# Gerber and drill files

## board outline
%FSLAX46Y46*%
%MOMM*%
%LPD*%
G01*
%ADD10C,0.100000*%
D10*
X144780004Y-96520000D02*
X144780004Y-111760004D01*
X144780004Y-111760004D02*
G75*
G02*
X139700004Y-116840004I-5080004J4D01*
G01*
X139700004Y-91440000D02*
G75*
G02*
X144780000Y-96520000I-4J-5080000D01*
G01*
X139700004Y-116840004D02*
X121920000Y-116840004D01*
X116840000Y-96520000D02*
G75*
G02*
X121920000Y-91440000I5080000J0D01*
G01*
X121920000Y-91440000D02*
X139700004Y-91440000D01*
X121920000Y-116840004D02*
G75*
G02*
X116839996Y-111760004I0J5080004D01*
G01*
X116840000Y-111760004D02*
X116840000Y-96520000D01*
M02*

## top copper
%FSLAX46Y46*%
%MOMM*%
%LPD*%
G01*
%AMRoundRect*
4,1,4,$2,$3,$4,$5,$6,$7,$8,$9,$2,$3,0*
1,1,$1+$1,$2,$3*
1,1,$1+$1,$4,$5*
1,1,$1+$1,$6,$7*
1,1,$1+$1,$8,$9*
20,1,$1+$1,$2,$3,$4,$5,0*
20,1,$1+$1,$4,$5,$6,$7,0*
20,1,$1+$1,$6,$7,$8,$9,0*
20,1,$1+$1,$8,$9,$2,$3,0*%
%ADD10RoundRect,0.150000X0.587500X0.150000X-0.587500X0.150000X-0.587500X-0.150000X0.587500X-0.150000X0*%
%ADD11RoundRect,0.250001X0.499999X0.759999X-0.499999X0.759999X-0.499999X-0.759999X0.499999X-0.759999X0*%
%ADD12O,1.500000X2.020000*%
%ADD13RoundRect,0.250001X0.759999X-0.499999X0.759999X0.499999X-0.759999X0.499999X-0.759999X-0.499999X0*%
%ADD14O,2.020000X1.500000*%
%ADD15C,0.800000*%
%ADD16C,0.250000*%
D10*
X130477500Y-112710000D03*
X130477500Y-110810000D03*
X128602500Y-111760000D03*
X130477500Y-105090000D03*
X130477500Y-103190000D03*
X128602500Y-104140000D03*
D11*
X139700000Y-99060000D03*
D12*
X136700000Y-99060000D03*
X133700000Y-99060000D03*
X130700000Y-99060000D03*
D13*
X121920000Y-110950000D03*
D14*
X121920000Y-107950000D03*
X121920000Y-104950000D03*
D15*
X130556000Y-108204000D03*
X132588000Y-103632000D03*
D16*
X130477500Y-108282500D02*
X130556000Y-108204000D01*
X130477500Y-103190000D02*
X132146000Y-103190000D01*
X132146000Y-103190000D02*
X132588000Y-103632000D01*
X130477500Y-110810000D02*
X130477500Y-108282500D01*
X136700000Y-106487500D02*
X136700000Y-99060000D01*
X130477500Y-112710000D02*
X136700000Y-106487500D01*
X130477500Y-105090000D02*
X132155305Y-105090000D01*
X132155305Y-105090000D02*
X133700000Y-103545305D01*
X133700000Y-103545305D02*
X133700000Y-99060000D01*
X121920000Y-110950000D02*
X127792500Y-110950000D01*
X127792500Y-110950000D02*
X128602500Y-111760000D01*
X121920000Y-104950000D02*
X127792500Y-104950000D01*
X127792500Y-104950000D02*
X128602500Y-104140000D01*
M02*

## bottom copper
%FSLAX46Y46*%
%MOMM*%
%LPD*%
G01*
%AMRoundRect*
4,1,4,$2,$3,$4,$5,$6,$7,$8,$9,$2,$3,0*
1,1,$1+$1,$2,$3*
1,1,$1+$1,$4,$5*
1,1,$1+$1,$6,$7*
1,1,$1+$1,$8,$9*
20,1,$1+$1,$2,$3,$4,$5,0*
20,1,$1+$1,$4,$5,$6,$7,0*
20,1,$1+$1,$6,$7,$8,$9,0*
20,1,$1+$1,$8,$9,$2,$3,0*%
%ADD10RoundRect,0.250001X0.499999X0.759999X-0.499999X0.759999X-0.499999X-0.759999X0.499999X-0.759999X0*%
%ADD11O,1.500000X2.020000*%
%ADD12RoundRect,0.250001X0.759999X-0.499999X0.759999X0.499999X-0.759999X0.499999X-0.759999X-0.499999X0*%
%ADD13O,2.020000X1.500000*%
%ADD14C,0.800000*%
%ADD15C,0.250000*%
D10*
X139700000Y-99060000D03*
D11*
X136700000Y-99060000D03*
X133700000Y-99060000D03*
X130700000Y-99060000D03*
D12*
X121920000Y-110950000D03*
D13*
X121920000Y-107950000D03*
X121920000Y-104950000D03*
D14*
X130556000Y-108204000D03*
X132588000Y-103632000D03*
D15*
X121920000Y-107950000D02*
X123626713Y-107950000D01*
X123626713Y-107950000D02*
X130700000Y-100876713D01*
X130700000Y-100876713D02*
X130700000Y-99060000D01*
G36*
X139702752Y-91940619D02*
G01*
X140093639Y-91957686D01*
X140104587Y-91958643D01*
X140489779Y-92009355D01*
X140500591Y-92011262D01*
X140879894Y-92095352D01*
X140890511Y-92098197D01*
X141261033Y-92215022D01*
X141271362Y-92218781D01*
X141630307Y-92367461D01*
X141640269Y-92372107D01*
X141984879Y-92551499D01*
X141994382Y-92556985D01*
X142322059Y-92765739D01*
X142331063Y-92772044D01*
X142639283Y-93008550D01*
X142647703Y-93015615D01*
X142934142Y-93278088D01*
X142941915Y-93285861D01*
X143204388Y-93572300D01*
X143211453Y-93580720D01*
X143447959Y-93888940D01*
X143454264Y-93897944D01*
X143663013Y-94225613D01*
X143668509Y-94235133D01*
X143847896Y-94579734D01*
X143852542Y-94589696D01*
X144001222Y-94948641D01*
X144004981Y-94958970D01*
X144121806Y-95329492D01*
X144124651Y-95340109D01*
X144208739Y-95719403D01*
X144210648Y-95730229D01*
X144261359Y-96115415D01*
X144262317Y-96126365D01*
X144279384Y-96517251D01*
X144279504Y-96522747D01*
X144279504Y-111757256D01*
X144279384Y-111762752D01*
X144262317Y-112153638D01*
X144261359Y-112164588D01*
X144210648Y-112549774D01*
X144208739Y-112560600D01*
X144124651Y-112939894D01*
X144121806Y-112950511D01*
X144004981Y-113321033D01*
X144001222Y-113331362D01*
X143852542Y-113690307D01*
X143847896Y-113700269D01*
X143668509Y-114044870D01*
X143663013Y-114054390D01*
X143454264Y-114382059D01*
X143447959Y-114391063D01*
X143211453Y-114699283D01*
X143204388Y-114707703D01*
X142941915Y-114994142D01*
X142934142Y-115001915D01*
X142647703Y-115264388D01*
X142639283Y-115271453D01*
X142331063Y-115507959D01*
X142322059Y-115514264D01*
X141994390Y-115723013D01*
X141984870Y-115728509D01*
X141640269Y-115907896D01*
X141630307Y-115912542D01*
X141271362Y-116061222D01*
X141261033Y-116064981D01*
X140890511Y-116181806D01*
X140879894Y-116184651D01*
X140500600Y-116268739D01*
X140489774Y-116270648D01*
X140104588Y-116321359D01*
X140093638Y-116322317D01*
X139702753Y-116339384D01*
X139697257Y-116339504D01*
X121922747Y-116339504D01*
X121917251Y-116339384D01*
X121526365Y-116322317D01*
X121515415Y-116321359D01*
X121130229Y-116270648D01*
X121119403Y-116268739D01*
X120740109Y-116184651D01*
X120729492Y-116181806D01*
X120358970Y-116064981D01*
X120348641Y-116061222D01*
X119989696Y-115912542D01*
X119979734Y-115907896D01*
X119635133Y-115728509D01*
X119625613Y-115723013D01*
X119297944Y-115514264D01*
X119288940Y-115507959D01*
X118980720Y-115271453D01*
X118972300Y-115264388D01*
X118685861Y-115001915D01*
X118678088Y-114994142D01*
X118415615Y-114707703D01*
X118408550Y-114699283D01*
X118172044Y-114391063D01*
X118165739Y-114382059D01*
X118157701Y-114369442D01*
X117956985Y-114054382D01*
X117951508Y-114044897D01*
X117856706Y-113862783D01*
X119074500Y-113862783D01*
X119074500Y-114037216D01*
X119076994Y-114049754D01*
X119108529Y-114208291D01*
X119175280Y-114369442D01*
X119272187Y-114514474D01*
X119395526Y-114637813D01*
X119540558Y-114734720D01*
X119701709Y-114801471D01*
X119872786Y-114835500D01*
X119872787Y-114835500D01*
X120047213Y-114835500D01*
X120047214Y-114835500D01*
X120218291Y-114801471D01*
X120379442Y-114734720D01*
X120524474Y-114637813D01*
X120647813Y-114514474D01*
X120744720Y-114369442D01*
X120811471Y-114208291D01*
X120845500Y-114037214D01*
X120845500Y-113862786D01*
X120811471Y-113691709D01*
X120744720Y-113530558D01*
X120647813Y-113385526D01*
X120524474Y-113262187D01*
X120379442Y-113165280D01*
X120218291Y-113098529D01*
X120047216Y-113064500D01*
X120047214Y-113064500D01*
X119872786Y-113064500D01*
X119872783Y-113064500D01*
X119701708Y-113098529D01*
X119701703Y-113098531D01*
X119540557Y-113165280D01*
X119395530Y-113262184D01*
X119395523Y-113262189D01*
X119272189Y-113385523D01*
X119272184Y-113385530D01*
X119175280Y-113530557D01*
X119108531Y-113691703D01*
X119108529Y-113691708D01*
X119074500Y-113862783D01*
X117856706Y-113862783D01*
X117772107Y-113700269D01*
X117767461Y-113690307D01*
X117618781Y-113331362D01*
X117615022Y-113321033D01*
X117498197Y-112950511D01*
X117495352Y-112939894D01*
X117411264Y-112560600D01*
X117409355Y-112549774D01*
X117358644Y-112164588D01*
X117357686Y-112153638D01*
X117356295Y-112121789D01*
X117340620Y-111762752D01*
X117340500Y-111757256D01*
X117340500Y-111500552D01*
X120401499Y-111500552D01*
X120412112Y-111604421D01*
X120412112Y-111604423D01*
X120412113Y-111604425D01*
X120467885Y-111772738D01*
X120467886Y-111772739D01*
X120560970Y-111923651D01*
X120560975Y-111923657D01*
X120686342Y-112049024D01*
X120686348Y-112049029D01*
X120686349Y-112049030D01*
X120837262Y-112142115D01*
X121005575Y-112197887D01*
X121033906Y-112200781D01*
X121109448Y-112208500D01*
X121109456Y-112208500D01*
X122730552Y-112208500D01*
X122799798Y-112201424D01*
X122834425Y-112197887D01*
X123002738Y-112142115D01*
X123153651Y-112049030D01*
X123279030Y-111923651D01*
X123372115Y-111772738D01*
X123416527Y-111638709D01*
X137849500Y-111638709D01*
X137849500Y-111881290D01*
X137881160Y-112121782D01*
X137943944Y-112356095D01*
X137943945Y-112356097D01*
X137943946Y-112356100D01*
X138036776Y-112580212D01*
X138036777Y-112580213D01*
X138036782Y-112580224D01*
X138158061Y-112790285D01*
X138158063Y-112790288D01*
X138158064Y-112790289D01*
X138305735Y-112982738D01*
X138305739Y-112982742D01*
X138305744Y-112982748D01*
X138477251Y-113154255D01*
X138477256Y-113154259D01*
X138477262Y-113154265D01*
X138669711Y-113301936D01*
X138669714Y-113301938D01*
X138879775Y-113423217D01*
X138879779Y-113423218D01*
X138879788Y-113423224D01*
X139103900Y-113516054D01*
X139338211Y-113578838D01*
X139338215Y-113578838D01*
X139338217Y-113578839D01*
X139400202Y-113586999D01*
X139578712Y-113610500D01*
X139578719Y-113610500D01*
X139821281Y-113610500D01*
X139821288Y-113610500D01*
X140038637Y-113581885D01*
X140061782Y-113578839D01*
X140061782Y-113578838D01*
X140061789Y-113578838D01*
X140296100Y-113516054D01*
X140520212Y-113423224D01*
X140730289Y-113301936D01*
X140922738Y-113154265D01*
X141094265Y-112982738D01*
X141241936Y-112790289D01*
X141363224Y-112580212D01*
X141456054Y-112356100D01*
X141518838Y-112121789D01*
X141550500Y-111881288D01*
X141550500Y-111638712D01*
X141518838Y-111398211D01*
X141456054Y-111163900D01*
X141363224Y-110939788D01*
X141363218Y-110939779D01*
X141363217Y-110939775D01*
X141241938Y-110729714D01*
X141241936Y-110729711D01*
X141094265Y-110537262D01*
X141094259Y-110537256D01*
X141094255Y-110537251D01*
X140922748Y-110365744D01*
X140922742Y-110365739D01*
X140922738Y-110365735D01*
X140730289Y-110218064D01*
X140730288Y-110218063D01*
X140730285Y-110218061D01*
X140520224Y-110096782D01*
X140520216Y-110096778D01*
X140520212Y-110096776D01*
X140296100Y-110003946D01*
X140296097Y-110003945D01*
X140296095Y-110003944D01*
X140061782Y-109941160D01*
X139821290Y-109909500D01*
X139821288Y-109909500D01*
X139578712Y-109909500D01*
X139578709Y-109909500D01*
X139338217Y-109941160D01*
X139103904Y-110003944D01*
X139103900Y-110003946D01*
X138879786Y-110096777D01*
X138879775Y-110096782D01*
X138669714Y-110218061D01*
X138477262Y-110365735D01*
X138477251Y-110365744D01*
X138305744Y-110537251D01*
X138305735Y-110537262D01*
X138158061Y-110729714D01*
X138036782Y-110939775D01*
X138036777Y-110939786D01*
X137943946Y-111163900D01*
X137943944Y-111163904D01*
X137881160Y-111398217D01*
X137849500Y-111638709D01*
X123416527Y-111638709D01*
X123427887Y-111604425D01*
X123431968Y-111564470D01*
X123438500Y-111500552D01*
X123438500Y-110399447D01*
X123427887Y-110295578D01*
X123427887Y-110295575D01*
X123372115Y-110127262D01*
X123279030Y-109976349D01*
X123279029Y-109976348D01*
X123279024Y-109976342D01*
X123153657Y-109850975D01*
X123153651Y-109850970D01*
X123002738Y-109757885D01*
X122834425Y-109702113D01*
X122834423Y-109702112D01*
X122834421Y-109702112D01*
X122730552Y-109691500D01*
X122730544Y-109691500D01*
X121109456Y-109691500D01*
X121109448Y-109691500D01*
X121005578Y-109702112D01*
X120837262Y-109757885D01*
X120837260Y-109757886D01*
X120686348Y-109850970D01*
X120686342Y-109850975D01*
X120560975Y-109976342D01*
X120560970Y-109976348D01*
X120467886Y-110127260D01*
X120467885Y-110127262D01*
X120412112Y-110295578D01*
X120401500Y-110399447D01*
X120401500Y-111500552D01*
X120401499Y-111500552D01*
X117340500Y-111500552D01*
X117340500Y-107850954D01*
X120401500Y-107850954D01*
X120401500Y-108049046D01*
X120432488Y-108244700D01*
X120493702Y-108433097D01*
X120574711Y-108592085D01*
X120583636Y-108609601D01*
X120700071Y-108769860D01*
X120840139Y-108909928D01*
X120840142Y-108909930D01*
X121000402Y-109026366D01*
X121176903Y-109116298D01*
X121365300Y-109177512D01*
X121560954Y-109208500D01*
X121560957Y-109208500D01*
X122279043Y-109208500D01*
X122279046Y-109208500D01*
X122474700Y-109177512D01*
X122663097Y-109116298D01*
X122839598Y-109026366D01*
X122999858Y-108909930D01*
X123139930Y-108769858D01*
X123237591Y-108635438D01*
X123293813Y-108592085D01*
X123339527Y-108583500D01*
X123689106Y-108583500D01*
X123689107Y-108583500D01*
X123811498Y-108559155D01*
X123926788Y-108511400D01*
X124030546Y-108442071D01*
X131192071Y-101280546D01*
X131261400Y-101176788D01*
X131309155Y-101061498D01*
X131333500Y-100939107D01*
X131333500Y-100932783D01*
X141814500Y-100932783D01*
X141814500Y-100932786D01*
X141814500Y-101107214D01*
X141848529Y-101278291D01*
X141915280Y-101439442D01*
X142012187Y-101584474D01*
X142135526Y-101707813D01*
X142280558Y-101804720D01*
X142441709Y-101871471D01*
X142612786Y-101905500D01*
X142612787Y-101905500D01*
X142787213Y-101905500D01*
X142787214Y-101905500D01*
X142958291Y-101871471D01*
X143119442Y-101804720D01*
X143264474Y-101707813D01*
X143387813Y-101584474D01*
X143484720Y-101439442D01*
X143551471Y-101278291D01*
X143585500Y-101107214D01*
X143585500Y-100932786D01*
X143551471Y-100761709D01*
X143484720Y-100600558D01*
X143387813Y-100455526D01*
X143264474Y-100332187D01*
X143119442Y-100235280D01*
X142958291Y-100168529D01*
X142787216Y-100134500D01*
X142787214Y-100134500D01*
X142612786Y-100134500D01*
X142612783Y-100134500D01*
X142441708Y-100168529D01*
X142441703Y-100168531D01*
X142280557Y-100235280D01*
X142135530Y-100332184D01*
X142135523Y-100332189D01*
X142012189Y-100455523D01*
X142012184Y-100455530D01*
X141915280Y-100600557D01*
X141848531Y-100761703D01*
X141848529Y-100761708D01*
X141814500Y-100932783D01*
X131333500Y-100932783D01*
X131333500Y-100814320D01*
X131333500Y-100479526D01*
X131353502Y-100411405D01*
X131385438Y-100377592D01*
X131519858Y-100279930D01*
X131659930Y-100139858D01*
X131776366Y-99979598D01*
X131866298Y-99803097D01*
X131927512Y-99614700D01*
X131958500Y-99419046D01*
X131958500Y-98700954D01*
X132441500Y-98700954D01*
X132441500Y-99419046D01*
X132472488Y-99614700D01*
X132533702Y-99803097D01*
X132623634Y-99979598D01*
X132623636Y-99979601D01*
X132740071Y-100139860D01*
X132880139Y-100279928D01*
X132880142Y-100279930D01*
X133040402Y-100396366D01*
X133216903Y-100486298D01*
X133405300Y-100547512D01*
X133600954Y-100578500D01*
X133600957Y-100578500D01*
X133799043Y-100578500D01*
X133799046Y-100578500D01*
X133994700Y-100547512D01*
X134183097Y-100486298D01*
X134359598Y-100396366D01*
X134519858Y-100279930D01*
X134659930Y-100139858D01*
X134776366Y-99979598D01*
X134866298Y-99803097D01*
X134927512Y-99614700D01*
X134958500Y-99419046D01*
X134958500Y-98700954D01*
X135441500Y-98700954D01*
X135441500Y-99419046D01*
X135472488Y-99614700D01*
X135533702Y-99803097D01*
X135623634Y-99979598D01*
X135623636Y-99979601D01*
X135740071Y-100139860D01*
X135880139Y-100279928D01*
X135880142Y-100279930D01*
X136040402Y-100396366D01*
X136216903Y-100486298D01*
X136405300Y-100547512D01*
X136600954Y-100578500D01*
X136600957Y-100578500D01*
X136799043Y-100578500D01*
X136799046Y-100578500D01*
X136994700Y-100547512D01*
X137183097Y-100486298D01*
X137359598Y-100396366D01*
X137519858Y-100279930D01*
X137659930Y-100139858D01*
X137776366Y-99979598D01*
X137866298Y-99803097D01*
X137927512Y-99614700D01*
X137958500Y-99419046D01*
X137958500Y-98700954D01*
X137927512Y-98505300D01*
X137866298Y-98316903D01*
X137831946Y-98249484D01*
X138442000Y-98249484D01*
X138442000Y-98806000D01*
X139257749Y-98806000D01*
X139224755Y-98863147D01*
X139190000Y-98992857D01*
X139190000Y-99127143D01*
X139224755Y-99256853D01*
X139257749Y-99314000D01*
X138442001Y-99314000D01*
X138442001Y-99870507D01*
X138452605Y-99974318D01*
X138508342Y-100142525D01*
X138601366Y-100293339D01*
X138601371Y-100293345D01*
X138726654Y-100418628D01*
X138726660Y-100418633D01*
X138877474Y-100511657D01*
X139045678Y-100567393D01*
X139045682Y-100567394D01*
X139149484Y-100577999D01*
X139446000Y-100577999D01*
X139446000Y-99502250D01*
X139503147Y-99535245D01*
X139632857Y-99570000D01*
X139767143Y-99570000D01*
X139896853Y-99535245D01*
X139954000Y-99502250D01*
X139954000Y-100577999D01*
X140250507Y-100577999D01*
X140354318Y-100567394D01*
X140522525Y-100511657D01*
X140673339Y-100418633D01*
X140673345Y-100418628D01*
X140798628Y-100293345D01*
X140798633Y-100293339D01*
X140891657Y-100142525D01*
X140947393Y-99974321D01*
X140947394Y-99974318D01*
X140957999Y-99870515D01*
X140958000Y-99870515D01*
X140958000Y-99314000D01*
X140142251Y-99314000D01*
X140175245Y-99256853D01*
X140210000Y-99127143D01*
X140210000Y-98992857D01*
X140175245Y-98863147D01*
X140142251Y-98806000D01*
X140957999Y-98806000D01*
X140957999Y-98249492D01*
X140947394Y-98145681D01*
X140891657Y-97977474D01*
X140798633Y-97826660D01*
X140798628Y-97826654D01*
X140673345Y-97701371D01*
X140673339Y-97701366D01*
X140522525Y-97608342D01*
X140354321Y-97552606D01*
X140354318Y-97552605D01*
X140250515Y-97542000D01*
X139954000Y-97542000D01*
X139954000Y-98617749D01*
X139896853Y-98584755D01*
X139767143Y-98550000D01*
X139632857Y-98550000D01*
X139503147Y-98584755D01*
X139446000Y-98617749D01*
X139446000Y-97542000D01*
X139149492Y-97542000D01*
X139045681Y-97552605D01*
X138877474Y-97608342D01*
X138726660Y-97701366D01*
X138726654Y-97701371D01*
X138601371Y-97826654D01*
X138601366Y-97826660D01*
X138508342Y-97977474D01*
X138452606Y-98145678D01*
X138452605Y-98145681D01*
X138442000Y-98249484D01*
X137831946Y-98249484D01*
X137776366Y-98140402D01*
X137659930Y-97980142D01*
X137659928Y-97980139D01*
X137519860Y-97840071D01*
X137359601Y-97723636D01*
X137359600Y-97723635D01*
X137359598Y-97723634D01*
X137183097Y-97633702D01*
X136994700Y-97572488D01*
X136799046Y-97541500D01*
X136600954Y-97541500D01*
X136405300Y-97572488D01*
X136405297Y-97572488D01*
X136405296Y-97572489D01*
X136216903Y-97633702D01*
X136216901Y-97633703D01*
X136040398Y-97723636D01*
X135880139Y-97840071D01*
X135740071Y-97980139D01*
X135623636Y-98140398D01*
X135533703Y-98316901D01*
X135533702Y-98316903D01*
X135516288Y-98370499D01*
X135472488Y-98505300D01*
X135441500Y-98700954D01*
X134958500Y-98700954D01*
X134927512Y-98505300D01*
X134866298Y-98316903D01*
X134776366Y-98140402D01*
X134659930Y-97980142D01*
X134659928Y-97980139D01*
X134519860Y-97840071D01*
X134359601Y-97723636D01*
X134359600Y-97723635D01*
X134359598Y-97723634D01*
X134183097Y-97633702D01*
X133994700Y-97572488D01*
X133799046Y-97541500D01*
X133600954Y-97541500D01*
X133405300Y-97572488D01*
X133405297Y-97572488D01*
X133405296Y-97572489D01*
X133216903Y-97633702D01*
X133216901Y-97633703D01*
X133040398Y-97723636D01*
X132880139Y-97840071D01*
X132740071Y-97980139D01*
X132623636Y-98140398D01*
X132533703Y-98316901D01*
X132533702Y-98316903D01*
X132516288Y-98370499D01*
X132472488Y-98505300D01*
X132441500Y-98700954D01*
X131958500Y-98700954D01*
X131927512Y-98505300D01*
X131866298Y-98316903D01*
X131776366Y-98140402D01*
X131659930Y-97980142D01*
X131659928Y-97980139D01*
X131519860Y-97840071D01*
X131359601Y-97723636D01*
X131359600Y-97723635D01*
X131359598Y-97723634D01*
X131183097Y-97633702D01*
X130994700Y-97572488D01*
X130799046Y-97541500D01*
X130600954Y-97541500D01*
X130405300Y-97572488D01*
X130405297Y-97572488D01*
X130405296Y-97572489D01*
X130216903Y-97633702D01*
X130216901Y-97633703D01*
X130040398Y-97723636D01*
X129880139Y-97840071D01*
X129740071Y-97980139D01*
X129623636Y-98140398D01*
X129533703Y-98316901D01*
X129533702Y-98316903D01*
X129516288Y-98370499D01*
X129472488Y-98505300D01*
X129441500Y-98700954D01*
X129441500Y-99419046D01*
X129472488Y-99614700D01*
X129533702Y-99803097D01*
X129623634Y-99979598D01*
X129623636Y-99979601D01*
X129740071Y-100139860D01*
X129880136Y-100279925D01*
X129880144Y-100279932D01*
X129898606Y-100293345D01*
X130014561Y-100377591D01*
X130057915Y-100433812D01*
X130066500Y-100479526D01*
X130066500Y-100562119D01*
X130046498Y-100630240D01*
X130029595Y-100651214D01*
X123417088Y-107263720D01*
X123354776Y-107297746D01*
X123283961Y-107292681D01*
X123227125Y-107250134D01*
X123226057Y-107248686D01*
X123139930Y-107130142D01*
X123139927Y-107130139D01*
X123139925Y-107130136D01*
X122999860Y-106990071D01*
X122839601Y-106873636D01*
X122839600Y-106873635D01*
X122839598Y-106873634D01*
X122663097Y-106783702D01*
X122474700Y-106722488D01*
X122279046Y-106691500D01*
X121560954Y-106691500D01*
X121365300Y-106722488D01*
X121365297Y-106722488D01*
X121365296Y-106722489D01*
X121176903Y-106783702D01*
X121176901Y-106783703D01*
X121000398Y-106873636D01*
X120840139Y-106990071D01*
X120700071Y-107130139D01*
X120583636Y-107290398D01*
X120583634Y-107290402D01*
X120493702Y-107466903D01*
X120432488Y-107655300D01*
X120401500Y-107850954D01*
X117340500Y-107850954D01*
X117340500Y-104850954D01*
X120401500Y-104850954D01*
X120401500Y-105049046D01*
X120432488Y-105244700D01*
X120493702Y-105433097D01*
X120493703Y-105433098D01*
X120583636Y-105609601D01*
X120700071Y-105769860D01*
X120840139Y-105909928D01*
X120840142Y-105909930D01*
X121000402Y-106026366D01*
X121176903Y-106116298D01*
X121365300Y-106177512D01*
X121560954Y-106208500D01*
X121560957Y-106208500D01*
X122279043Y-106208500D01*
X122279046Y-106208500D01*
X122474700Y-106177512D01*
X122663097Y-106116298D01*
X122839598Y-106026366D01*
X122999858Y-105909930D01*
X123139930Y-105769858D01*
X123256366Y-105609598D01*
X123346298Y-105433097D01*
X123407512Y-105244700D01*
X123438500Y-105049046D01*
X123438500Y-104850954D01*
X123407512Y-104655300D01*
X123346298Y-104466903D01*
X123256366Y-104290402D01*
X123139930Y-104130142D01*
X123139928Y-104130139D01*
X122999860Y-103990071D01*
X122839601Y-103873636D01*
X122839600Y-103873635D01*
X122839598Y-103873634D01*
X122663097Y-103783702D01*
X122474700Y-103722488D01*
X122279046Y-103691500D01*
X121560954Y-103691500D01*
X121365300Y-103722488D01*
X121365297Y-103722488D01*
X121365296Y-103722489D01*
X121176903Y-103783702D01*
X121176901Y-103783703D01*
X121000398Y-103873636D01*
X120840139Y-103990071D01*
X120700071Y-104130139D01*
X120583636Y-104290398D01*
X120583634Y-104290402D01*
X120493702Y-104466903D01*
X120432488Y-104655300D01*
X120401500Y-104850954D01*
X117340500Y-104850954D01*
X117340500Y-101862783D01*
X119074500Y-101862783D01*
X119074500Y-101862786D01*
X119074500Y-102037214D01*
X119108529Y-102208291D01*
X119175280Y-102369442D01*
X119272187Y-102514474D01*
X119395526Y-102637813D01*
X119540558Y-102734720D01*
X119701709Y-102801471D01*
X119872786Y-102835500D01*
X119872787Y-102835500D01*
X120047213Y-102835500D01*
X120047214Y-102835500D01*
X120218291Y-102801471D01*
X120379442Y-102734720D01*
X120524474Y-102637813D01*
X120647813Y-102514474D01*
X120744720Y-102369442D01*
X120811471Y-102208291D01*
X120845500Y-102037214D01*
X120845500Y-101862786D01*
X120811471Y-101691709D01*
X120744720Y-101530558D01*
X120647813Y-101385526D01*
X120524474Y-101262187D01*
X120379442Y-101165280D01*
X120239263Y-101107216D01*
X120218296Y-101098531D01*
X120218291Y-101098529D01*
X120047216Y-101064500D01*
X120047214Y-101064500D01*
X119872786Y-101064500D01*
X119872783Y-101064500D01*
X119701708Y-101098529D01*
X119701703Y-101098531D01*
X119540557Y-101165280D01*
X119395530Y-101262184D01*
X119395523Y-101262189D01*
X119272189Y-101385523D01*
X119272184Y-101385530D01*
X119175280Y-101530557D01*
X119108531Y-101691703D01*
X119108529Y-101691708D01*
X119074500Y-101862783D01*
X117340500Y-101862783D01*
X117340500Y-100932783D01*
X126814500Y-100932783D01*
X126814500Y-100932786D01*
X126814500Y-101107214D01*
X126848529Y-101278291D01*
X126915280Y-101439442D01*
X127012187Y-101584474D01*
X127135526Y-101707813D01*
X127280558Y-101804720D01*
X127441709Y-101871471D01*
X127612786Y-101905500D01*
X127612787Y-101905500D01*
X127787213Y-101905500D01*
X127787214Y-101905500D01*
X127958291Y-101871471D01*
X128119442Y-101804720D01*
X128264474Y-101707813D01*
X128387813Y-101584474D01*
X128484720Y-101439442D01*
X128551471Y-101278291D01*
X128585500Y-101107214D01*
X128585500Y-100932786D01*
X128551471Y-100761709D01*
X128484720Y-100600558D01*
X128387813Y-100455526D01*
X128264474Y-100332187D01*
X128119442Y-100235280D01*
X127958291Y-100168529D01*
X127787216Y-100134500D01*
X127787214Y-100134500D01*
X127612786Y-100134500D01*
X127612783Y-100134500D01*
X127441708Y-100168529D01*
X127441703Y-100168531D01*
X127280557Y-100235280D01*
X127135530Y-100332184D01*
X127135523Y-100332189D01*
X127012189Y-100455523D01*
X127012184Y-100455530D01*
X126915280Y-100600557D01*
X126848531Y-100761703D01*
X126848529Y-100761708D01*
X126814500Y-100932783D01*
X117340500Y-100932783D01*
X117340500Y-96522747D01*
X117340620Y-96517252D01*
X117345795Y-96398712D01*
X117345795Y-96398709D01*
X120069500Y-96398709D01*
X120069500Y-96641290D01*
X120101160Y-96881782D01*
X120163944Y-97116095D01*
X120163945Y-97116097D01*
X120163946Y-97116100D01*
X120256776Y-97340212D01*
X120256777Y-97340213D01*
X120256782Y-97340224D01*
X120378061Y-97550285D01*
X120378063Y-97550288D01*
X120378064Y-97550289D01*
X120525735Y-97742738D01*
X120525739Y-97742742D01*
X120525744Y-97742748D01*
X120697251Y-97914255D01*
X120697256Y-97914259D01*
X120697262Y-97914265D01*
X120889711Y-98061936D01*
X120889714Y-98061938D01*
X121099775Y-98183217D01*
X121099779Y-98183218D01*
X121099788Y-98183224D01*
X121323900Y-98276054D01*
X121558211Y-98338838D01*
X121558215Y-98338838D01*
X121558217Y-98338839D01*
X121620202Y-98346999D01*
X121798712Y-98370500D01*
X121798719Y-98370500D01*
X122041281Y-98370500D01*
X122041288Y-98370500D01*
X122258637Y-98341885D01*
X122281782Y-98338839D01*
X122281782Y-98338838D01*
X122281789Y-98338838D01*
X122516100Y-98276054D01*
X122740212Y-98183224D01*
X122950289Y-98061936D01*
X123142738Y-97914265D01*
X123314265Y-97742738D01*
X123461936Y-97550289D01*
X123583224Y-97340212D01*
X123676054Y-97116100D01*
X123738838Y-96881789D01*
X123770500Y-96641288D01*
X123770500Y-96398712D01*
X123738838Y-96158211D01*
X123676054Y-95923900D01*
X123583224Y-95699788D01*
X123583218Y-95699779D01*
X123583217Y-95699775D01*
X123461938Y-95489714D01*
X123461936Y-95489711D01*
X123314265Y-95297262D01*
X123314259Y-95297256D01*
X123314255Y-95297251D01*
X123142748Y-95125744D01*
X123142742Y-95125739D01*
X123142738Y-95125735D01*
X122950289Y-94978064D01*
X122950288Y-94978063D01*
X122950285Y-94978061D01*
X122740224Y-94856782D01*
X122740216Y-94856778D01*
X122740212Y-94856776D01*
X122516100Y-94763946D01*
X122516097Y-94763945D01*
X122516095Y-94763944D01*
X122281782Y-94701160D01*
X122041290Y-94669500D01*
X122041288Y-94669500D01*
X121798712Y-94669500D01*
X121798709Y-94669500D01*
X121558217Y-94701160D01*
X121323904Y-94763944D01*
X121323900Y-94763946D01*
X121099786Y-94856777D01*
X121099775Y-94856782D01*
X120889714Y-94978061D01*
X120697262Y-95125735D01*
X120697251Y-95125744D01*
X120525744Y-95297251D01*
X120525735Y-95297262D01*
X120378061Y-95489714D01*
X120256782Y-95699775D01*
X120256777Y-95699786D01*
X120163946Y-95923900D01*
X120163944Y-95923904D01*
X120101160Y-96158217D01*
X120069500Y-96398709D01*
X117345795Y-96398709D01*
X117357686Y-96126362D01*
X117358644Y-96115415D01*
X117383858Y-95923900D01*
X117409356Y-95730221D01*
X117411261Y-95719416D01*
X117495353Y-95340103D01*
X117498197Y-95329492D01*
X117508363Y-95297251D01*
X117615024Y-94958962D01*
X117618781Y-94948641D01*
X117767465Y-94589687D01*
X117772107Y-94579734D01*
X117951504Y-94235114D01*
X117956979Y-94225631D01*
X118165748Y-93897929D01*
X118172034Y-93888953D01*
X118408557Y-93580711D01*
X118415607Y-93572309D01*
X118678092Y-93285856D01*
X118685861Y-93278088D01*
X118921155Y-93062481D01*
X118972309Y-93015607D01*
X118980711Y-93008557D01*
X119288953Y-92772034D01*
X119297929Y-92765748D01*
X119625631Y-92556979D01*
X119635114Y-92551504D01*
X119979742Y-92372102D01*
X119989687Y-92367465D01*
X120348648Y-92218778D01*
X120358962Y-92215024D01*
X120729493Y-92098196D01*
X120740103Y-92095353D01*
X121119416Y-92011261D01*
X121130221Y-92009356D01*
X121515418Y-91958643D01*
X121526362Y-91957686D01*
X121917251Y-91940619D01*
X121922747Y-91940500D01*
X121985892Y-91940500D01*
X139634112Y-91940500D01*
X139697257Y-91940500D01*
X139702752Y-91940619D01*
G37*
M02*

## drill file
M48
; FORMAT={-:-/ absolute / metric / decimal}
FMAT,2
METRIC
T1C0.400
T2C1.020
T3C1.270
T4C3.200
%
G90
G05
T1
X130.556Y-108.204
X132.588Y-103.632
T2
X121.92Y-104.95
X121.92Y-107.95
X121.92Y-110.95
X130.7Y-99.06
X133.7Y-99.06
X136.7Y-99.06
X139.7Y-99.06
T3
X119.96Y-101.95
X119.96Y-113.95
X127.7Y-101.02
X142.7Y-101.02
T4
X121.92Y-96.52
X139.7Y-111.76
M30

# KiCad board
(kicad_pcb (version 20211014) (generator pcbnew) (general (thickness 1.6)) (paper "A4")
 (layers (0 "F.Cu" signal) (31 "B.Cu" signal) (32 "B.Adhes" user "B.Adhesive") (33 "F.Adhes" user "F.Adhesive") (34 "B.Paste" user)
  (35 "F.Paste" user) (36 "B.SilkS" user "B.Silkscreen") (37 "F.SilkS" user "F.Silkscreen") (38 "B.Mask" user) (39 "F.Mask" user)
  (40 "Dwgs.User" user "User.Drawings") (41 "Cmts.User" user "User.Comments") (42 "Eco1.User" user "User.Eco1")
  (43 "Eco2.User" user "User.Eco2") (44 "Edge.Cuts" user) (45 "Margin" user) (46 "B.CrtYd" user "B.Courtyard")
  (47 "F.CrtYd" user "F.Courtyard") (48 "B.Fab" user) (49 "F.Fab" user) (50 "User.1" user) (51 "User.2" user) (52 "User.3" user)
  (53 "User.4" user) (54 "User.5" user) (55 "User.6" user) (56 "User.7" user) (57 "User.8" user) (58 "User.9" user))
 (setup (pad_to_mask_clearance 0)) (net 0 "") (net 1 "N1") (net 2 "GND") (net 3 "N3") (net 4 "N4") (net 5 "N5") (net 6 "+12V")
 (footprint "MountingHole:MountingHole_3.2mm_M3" (layer "F.Cu") (at 139.7 111.76)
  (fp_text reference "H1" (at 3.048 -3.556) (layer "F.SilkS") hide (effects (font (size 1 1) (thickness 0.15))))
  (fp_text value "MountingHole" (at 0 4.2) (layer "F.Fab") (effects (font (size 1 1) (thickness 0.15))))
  (pad "" np_thru_hole circle (at 0 0) (size 3.2 3.2) (drill 3.2) (layers *.Cu *.Mask)))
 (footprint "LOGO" (layer "F.Cu") (at 139.3698 105.0036)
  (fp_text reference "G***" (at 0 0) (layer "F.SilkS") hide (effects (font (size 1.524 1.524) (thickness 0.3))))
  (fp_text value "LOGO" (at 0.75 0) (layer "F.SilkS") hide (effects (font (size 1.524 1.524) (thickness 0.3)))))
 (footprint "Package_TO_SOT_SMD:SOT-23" (layer "F.Cu") (at 129.54 111.76 180)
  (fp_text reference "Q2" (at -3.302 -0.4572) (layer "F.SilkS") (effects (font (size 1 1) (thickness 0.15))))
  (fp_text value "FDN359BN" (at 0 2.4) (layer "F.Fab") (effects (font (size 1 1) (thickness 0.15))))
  (pad "1" smd roundrect (at -0.9375 -0.95 180) (size 1.475 0.6) (layers "F.Cu" "F.Paste" "F.Mask") (roundrect_rratio 0.25) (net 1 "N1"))
  (pad "2" smd roundrect (at -0.9375 0.95 180) (size 1.475 0.6) (layers "F.Cu" "F.Paste" "F.Mask") (roundrect_rratio 0.25) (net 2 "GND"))
  (pad "3" smd roundrect (at 0.9375 0 180) (size 1.475 0.6) (layers "F.Cu" "F.Paste" "F.Mask") (roundrect_rratio 0.25) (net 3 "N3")))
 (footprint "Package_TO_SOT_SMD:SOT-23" (layer "F.Cu") (at 129.54 104.14 180)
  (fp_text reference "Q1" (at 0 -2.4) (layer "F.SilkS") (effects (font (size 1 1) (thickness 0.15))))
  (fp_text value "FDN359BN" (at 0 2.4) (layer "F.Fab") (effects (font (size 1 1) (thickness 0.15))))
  (pad "1" smd roundrect (at -0.9375 -0.95 180) (size 1.475 0.6) (layers "F.Cu" "F.Paste" "F.Mask") (roundrect_rratio 0.25) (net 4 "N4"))
  (pad "2" smd roundrect (at -0.9375 0.95 180) (size 1.475 0.6) (layers "F.Cu" "F.Paste" "F.Mask") (roundrect_rratio 0.25) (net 2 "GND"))
  (pad "3" smd roundrect (at 0.9375 0 180) (size 1.475 0.6) (layers "F.Cu" "F.Paste" "F.Mask") (roundrect_rratio 0.25) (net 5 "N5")))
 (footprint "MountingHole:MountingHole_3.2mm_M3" (layer "F.Cu") (at 121.92 96.52)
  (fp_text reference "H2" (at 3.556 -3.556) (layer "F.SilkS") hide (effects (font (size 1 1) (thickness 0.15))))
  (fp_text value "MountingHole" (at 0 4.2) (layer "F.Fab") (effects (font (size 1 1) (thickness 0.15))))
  (pad "" np_thru_hole circle (at 0 0) (size 3.2 3.2) (drill 3.2) (layers *.Cu *.Mask)))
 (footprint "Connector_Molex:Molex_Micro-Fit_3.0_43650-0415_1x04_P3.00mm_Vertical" (layer "F.Cu") (at 139.7 99.06 180)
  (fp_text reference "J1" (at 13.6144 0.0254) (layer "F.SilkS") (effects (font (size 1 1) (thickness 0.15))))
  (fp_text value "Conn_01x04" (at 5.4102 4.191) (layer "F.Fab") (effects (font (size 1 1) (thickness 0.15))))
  (pad "" np_thru_hole circle (at 12 -1.96 180) (size 1.27 1.27) (drill 1.27) (layers *.Cu *.Mask))
  (pad "" np_thru_hole circle (at -3 -1.96 180) (size 1.27 1.27) (drill 1.27) (layers *.Cu *.Mask))
  (pad "1" thru_hole roundrect (at 0 0 180) (size 1.5 2.02) (drill 1.02) (layers *.Cu *.Mask) (roundrect_rratio 0.166667) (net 2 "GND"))
  (pad "2" thru_hole oval (at 3 0 180) (size 1.5 2.02) (drill 1.02) (layers *.Cu *.Mask) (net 1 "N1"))
  (pad "3" thru_hole oval (at 6 0 180) (size 1.5 2.02) (drill 1.02) (layers *.Cu *.Mask) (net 4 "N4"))
  (pad "4" thru_hole oval (at 9 0 180) (size 1.5 2.02) (drill 1.02) (layers *.Cu *.Mask) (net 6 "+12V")))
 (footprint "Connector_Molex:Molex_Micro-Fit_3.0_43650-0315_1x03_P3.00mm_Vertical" (layer "F.Cu") (at 121.92 110.95 90)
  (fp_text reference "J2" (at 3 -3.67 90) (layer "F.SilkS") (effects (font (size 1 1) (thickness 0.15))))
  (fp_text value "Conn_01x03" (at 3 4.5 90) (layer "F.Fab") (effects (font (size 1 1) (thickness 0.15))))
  (pad "" np_thru_hole circle (at 9 -1.96 90) (size 1.27 1.27) (drill 1.27) (layers *.Cu *.Mask))
  (pad "" np_thru_hole circle (at -3 -1.96 90) (size 1.27 1.27) (drill 1.27) (layers *.Cu *.Mask))
  (pad "1" thru_hole roundrect (at 0 0 90) (size 1.5 2.02) (drill 1.02) (layers *.Cu *.Mask) (roundrect_rratio 0.166667) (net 3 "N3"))
  (pad "2" thru_hole oval (at 3 0 90) (size 1.5 2.02) (drill 1.02) (layers *.Cu *.Mask) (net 6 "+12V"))
  (pad "3" thru_hole oval (at 6 0 90) (size 1.5 2.02) (drill 1.02) (layers *.Cu *.Mask) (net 5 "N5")))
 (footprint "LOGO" (layer "F.Cu") (at 134.9798 93.9588)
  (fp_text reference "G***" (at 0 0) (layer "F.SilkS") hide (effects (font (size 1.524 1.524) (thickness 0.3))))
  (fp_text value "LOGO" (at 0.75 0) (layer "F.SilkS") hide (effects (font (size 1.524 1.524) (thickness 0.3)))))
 (gr_line (start 144.780004 96.52) (end 144.780004 111.760004) (layer "Edge.Cuts") (width 0.1))
 (gr_arc (start 144.780004 111.760004) (mid 143.292106 115.352106) (end 139.700004 116.840004) (layer "Edge.Cuts") (width 0.1))
 (gr_arc (start 139.700004 91.44) (mid 143.292106 92.927898) (end 144.780004 96.52) (layer "Edge.Cuts") (width 0.1))
 (gr_line (start 139.700004 116.840004) (end 121.92 116.840004) (layer "Edge.Cuts") (width 0.1))
 (gr_arc (start 116.84 96.52) (mid 118.327898 92.927898) (end 121.92 91.44) (layer "Edge.Cuts") (width 0.1))
 (gr_line (start 121.92 91.44) (end 139.700004 91.44) (layer "Edge.Cuts") (width 0.1))
 (gr_arc (start 121.92 116.840004) (mid 118.327898 115.352106) (end 116.84 111.760004) (layer "Edge.Cuts") (width 0.1))
 (gr_line (start 116.84 111.760004) (end 116.84 96.52) (layer "Edge.Cuts") (width 0.1))
 (segment (start 130.4775 108.2825) (end 130.556 108.204) (width 0.25) (layer "F.Cu") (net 2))
 (segment (start 130.4775 103.19) (end 132.146 103.19) (width 0.25) (layer "F.Cu") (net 2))
 (segment (start 132.146 103.19) (end 132.588 103.632) (width 0.25) (layer "F.Cu") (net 2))
 (segment (start 130.4775 110.81) (end 130.4775 108.2825) (width 0.25) (layer "F.Cu") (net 2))
 (via (at 130.556 108.204) (size 0.8) (drill 0.4) (layers "F.Cu" "B.Cu") (free) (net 2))
 (via (at 132.588 103.632) (size 0.8) (drill 0.4) (layers "F.Cu" "B.Cu") (free) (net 2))
 (segment (start 136.7 106.4875) (end 136.7 99.06) (width 0.25) (layer "F.Cu") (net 1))
 (segment (start 130.4775 112.71) (end 136.7 106.4875) (width 0.25) (layer "F.Cu") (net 1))
 (segment (start 130.4775 105.09) (end 132.155305 105.09) (width 0.25) (layer "F.Cu") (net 4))
 (segment (start 132.155305 105.09) (end 133.7 103.545305) (width 0.25) (layer "F.Cu") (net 4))
 (segment (start 133.7 103.545305) (end 133.7 99.06) (width 0.25) (layer "F.Cu") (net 4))
 (segment (start 121.92 107.95) (end 123.626713 107.95) (width 0.25) (layer "B.Cu") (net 6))
 (segment (start 123.626713 107.95) (end 130.7 100.876713) (width 0.25) (layer "B.Cu") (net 6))
 (segment (start 130.7 100.876713) (end 130.7 99.06) (width 0.25) (layer "B.Cu") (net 6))
 (segment (start 121.92 110.95) (end 127.7925 110.95) (width 0.25) (layer "F.Cu") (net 3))
 (segment (start 127.7925 110.95) (end 128.6025 111.76) (width 0.25) (layer "F.Cu") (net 3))
 (segment (start 121.92 104.95) (end 127.7925 104.95) (width 0.25) (layer "F.Cu") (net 5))
 (segment (start 127.7925 104.95) (end 128.6025 104.14) (width 0.25) (layer "F.Cu") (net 5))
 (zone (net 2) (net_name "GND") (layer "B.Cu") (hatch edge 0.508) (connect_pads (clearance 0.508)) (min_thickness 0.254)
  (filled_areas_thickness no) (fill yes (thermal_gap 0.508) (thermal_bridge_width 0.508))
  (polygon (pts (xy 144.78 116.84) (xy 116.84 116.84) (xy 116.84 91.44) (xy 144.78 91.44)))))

